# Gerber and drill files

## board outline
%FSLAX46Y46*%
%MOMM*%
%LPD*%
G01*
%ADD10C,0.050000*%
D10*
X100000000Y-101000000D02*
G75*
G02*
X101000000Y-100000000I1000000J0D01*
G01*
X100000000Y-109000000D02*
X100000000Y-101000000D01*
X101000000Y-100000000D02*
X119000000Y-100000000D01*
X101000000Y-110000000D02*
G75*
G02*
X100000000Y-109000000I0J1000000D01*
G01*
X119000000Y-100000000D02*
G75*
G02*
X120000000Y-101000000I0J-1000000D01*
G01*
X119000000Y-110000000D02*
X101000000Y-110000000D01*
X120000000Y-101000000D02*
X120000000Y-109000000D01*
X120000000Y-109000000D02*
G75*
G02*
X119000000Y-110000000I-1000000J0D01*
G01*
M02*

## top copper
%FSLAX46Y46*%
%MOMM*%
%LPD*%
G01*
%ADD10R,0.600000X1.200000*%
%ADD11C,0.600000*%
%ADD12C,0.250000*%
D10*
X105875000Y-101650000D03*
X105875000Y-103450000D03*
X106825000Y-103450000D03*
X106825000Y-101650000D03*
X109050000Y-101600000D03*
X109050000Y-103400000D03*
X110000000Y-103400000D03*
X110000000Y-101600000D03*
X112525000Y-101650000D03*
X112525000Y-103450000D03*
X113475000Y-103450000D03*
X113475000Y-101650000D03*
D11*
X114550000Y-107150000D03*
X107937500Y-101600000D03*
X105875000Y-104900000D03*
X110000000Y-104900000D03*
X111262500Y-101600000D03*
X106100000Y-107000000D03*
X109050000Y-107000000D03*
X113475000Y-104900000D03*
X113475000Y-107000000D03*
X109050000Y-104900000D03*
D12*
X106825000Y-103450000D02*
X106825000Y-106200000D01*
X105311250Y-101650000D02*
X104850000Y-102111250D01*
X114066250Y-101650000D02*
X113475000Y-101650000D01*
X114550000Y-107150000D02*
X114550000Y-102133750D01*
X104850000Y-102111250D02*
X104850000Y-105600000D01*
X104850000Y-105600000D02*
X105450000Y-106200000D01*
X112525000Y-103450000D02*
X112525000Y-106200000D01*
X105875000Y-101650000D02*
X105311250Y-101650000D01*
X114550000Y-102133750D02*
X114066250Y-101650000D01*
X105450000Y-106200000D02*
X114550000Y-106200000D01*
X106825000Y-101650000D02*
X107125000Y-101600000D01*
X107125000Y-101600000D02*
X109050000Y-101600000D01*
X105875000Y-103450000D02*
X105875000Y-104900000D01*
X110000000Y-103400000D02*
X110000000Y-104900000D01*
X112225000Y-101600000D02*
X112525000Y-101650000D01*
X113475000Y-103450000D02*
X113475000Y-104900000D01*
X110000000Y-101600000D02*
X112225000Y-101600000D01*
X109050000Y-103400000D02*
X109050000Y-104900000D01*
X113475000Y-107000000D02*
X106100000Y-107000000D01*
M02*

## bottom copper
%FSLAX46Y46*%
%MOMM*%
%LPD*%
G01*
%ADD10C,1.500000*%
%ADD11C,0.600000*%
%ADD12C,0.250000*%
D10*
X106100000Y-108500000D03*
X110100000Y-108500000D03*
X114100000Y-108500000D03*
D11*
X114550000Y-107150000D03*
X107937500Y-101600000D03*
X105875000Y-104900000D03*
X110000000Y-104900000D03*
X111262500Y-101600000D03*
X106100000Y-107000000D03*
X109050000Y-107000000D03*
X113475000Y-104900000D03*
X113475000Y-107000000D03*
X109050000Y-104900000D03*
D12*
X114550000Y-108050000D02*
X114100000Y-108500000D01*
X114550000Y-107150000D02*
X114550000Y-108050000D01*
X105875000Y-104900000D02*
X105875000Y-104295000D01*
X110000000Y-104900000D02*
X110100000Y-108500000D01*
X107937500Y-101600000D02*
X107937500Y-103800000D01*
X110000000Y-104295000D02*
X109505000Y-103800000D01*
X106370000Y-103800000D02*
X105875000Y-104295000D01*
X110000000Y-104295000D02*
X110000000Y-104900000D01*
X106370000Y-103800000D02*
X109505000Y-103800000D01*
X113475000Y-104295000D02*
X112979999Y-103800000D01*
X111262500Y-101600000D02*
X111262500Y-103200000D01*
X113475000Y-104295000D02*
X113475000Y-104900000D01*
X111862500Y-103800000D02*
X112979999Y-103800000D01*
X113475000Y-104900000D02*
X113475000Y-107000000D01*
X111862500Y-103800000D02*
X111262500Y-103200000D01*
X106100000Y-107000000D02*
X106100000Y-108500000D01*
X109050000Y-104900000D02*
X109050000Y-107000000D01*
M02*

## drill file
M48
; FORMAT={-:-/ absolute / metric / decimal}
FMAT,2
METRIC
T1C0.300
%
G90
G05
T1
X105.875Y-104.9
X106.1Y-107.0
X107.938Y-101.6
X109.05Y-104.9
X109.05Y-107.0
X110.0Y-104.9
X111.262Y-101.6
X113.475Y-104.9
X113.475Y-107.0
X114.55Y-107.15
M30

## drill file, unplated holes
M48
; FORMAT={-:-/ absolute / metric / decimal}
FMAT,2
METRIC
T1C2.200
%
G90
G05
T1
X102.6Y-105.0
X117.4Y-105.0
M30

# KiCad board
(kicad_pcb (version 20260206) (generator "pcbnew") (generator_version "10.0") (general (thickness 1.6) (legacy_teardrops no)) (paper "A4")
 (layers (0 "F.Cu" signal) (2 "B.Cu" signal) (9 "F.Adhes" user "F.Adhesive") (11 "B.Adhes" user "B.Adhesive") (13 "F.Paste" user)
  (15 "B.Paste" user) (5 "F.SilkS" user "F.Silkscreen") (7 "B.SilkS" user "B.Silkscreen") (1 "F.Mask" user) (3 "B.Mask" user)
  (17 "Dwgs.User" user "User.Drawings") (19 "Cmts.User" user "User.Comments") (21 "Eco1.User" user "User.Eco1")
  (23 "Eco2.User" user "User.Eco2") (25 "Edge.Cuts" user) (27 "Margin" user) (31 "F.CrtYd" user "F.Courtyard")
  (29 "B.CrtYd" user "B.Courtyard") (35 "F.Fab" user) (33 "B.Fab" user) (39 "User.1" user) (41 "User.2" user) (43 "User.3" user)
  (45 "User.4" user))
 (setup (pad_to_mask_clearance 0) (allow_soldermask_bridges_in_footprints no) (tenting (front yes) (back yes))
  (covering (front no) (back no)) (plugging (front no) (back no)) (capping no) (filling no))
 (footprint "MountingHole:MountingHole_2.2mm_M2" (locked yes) (layer "F.Cu") (at 117.4 105)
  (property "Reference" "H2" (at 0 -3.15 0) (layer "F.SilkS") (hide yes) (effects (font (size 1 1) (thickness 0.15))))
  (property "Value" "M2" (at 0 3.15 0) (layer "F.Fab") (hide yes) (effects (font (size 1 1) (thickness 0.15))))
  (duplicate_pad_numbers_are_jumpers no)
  (pad "" np_thru_hole circle (at 0 0) (size 2.2 2.2) (drill 2.2) (layers "*.Cu" "*.Mask")))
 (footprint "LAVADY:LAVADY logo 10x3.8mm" (layer "F.Cu") (at 109.8 108)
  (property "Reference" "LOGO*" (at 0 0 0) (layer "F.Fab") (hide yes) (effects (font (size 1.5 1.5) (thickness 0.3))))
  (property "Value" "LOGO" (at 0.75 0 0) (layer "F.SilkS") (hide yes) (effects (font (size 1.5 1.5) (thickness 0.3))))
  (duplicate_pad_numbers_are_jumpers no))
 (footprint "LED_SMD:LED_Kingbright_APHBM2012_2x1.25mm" (layer "F.Cu") (at 106.35 102.55)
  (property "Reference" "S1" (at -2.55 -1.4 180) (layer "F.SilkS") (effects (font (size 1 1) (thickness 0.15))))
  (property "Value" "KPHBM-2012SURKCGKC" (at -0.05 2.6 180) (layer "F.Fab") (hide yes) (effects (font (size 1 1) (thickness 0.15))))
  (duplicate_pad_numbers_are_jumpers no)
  (pad "1" smd rect (at -0.475 -0.9 90) (size 1.2 0.6) (layers "F.Cu" "F.Mask" "F.Paste") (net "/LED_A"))
  (pad "2" smd rect (at -0.475 0.9 90) (size 1.2 0.6) (layers "F.Cu" "F.Mask" "F.Paste") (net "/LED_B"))
  (pad "3" smd rect (at 0.475 0.9 90) (size 1.2 0.6) (layers "F.Cu" "F.Mask" "F.Paste") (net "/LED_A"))
  (pad "4" smd rect (at 0.475 -0.9 90) (size 1.2 0.6) (layers "F.Cu" "F.Mask" "F.Paste") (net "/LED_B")))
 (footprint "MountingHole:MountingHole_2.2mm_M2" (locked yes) (layer "F.Cu") (at 102.6 105)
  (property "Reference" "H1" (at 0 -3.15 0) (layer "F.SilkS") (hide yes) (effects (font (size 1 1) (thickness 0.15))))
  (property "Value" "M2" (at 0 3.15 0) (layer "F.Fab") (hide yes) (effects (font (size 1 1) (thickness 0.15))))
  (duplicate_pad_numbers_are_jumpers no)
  (pad "" np_thru_hole circle (at 0 0) (size 2.2 2.2) (drill 2.2) (layers "*.Cu" "*.Mask")))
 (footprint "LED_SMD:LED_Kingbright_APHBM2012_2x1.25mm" (layer "F.Cu") (at 109.525 102.5)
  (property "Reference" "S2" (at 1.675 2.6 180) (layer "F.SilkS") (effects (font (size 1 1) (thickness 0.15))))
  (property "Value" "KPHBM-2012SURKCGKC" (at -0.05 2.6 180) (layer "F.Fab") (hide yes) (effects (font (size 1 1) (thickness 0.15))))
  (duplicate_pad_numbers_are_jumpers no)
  (pad "1" smd rect (at -0.475 -0.9 90) (size 1.2 0.6) (layers "F.Cu" "F.Mask" "F.Paste") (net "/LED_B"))
  (pad "2" smd rect (at -0.475 0.9 90) (size 1.2 0.6) (layers "F.Cu" "F.Mask" "F.Paste") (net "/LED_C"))
  (pad "3" smd rect (at 0.475 0.9 90) (size 1.2 0.6) (layers "F.Cu" "F.Mask" "F.Paste") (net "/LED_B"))
  (pad "4" smd rect (at 0.475 -0.9 90) (size 1.2 0.6) (layers "F.Cu" "F.Mask" "F.Paste") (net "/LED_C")))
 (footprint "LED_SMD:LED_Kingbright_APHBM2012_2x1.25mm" (layer "F.Cu") (at 113 102.55)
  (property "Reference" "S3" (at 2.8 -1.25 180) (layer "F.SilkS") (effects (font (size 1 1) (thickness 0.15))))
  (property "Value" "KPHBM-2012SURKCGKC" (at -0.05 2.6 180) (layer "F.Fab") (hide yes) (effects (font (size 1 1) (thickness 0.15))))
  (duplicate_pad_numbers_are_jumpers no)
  (pad "1" smd rect (at -0.475 -0.9 90) (size 1.2 0.6) (layers "F.Cu" "F.Mask" "F.Paste") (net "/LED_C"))
  (pad "2" smd rect (at -0.475 0.9 90) (size 1.2 0.6) (layers "F.Cu" "F.Mask" "F.Paste") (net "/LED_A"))
  (pad "3" smd rect (at 0.475 0.9 90) (size 1.2 0.6) (layers "F.Cu" "F.Mask" "F.Paste") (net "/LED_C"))
  (pad "4" smd rect (at 0.475 -0.9 90) (size 1.2 0.6) (layers "F.Cu" "F.Mask" "F.Paste") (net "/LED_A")))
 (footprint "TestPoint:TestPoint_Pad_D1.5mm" (layer "B.Cu") (at 106.1 108.5 180)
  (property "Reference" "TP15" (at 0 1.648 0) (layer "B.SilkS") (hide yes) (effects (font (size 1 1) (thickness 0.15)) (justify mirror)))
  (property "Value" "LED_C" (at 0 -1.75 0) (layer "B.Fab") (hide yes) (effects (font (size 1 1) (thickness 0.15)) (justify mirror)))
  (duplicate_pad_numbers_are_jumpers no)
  (pad "1" smd circle (at 0 0 180) (size 1.5 1.5) (layers "B.Cu" "B.Mask") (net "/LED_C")))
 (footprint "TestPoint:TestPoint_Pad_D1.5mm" (layer "B.Cu") (at 110.1 108.5 180)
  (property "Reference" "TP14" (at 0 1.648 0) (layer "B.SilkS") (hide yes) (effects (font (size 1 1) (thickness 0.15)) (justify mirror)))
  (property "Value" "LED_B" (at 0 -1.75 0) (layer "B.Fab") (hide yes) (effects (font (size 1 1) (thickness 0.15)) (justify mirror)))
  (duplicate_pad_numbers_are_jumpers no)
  (pad "1" smd circle (at 0 0 180) (size 1.5 1.5) (layers "B.Cu" "B.Mask") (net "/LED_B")))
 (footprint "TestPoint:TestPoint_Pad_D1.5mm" (layer "B.Cu") (at 114.1 108.5 180)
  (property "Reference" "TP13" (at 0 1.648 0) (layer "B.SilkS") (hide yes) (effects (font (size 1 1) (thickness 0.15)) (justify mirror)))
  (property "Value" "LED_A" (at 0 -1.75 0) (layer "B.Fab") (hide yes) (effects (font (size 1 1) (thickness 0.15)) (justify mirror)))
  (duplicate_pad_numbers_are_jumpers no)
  (pad "1" smd circle (at 0 0 180) (size 1.5 1.5) (layers "B.Cu" "B.Mask") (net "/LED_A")))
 (gr_arc (start 100 101) (mid 100.292893 100.292893) (end 101 100) (stroke (width 0.05) (type default)) (layer "Edge.Cuts"))
 (gr_line (start 100 109) (end 100 101) (stroke (width 0.05) (type default)) (layer "Edge.Cuts"))
 (gr_line (start 101 100) (end 119 100) (stroke (width 0.05) (type default)) (layer "Edge.Cuts"))
 (gr_arc (start 101 110) (mid 100.292893 109.707107) (end 100 109) (stroke (width 0.05) (type default)) (layer "Edge.Cuts"))
 (gr_arc (start 119 100) (mid 119.707107 100.292893) (end 120 101) (stroke (width 0.05) (type default)) (layer "Edge.Cuts"))
 (gr_line (start 119 110) (end 101 110) (stroke (width 0.05) (type default)) (layer "Edge.Cuts"))
 (gr_line (start 120 101) (end 120 109) (stroke (width 0.05) (type default)) (layer "Edge.Cuts"))
 (gr_arc (start 120 109) (mid 119.707107 109.707107) (end 119 110) (stroke (width 0.05) (type default)) (layer "Edge.Cuts"))
 (segment (start 106.825 103.45) (end 106.825 106.2) (width 0.25) (layer "F.Cu") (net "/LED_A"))
 (segment (start 105.31125 101.65) (end 104.85 102.11125) (width 0.25) (layer "F.Cu") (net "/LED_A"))
 (segment (start 114.06625 101.65) (end 113.475 101.65) (width 0.25) (layer "F.Cu") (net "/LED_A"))
 (segment (start 114.55 107.15) (end 114.55 102.13375) (width 0.25) (layer "F.Cu") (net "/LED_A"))
 (segment (start 104.85 102.11125) (end 104.85 105.6) (width 0.25) (layer "F.Cu") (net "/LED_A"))
 (segment (start 104.85 105.6) (end 105.45 106.2) (width 0.25) (layer "F.Cu") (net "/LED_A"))
 (segment (start 112.525 103.45) (end 112.525 106.2) (width 0.25) (layer "F.Cu") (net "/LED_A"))
 (segment (start 105.875 101.65) (end 105.31125 101.65) (width 0.25) (layer "F.Cu") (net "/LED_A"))
 (segment (start 114.55 102.13375) (end 114.06625 101.65) (width 0.25) (layer "F.Cu") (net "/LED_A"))
 (segment (start 105.45 106.2) (end 114.55 106.2) (width 0.25) (layer "F.Cu") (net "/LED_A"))
 (via (at 114.55 107.15) (size 0.6) (drill 0.3) (layers "F.Cu" "B.Cu") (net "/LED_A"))
 (segment (start 114.55 108.05) (end 114.1 108.5) (width 0.25) (layer "B.Cu") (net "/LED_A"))
 (segment (start 114.55 107.15) (end 114.55 108.05) (width 0.25) (layer "B.Cu") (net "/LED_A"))
 (segment (start 106.825 101.65) (end 107.125 101.6) (width 0.25) (layer "F.Cu") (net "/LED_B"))
 (segment (start 107.125 101.6) (end 109.05 101.6) (width 0.25) (layer "F.Cu") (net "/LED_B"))
 (segment (start 105.875 103.45) (end 105.875 104.9) (width 0.25) (layer "F.Cu") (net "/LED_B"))
 (segment (start 110 103.4) (end 110 104.9) (width 0.25) (layer "F.Cu") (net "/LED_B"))
 (via (at 107.9375 101.6) (size 0.6) (drill 0.3) (layers "F.Cu" "B.Cu") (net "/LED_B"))
 (via (at 105.875 104.9) (size 0.6) (drill 0.3) (layers "F.Cu" "B.Cu") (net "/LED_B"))
 (via (at 110 104.9) (size 0.6) (drill 0.3) (layers "F.Cu" "B.Cu") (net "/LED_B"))
 (segment (start 105.875 104.9) (end 105.875 104.295) (width 0.25) (layer "B.Cu") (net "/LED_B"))
 (segment (start 110 104.9) (end 110.1 108.5) (width 0.25) (layer "B.Cu") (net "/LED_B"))
 (segment (start 107.9375 101.6) (end 107.9375 103.8) (width 0.25) (layer "B.Cu") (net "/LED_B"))
 (segment (start 110 104.295) (end 109.505 103.8) (width 0.25) (layer "B.Cu") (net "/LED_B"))
 (segment (start 106.37 103.8) (end 105.875 104.295) (width 0.25) (layer "B.Cu") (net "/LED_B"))
 (segment (start 110 104.295) (end 110 104.9) (width 0.25) (layer "B.Cu") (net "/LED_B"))
 (segment (start 106.37 103.8) (end 109.505 103.8) (width 0.25) (layer "B.Cu") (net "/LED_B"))
 (segment (start 112.225 101.6) (end 112.525 101.65) (width 0.25) (layer "F.Cu") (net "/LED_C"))
 (segment (start 113.475 103.45) (end 113.475 104.9) (width 0.25) (layer "F.Cu") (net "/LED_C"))
 (segment (start 110 101.6) (end 112.225 101.6) (width 0.25) (layer "F.Cu") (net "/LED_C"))
 (segment (start 109.05 103.4) (end 109.05 104.9) (width 0.25) (layer "F.Cu") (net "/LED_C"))
 (segment (start 113.475 107) (end 106.1 107) (width 0.25) (layer "F.Cu") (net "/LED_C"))
 (via (at 111.2625 101.6) (size 0.6) (drill 0.3) (layers "F.Cu" "B.Cu") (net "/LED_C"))
 (via (at 106.1 107) (size 0.6) (drill 0.3) (layers "F.Cu" "B.Cu") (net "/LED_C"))
 (via (at 109.05 107) (size 0.6) (drill 0.3) (layers "F.Cu" "B.Cu") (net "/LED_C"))
 (via (at 113.475 104.9) (size 0.6) (drill 0.3) (layers "F.Cu" "B.Cu") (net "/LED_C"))
 (via (at 113.475 107) (size 0.6) (drill 0.3) (layers "F.Cu" "B.Cu") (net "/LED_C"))
 (via (at 109.05 104.9) (size 0.6) (drill 0.3) (layers "F.Cu" "B.Cu") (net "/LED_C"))
 (segment (start 113.475 104.295) (end 112.979999 103.8) (width 0.25) (layer "B.Cu") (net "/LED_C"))
 (segment (start 111.2625 101.6) (end 111.2625 103.2) (width 0.25) (layer "B.Cu") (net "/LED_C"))
 (segment (start 113.475 104.295) (end 113.475 104.9) (width 0.25) (layer "B.Cu") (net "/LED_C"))
 (segment (start 111.8625 103.8) (end 112.979999 103.8) (width 0.25) (layer "B.Cu") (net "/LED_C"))
 (segment (start 113.475 104.9) (end 113.475 107) (width 0.25) (layer "B.Cu") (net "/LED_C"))
 (segment (start 111.8625 103.8) (end 111.2625 103.2) (width 0.25) (layer "B.Cu") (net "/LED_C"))
 (segment (start 106.1 107) (end 106.1 108.5) (width 0.25) (layer "B.Cu") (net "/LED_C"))
 (segment (start 109.05 104.9) (end 109.05 107) (width 0.25) (layer "B.Cu") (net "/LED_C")))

